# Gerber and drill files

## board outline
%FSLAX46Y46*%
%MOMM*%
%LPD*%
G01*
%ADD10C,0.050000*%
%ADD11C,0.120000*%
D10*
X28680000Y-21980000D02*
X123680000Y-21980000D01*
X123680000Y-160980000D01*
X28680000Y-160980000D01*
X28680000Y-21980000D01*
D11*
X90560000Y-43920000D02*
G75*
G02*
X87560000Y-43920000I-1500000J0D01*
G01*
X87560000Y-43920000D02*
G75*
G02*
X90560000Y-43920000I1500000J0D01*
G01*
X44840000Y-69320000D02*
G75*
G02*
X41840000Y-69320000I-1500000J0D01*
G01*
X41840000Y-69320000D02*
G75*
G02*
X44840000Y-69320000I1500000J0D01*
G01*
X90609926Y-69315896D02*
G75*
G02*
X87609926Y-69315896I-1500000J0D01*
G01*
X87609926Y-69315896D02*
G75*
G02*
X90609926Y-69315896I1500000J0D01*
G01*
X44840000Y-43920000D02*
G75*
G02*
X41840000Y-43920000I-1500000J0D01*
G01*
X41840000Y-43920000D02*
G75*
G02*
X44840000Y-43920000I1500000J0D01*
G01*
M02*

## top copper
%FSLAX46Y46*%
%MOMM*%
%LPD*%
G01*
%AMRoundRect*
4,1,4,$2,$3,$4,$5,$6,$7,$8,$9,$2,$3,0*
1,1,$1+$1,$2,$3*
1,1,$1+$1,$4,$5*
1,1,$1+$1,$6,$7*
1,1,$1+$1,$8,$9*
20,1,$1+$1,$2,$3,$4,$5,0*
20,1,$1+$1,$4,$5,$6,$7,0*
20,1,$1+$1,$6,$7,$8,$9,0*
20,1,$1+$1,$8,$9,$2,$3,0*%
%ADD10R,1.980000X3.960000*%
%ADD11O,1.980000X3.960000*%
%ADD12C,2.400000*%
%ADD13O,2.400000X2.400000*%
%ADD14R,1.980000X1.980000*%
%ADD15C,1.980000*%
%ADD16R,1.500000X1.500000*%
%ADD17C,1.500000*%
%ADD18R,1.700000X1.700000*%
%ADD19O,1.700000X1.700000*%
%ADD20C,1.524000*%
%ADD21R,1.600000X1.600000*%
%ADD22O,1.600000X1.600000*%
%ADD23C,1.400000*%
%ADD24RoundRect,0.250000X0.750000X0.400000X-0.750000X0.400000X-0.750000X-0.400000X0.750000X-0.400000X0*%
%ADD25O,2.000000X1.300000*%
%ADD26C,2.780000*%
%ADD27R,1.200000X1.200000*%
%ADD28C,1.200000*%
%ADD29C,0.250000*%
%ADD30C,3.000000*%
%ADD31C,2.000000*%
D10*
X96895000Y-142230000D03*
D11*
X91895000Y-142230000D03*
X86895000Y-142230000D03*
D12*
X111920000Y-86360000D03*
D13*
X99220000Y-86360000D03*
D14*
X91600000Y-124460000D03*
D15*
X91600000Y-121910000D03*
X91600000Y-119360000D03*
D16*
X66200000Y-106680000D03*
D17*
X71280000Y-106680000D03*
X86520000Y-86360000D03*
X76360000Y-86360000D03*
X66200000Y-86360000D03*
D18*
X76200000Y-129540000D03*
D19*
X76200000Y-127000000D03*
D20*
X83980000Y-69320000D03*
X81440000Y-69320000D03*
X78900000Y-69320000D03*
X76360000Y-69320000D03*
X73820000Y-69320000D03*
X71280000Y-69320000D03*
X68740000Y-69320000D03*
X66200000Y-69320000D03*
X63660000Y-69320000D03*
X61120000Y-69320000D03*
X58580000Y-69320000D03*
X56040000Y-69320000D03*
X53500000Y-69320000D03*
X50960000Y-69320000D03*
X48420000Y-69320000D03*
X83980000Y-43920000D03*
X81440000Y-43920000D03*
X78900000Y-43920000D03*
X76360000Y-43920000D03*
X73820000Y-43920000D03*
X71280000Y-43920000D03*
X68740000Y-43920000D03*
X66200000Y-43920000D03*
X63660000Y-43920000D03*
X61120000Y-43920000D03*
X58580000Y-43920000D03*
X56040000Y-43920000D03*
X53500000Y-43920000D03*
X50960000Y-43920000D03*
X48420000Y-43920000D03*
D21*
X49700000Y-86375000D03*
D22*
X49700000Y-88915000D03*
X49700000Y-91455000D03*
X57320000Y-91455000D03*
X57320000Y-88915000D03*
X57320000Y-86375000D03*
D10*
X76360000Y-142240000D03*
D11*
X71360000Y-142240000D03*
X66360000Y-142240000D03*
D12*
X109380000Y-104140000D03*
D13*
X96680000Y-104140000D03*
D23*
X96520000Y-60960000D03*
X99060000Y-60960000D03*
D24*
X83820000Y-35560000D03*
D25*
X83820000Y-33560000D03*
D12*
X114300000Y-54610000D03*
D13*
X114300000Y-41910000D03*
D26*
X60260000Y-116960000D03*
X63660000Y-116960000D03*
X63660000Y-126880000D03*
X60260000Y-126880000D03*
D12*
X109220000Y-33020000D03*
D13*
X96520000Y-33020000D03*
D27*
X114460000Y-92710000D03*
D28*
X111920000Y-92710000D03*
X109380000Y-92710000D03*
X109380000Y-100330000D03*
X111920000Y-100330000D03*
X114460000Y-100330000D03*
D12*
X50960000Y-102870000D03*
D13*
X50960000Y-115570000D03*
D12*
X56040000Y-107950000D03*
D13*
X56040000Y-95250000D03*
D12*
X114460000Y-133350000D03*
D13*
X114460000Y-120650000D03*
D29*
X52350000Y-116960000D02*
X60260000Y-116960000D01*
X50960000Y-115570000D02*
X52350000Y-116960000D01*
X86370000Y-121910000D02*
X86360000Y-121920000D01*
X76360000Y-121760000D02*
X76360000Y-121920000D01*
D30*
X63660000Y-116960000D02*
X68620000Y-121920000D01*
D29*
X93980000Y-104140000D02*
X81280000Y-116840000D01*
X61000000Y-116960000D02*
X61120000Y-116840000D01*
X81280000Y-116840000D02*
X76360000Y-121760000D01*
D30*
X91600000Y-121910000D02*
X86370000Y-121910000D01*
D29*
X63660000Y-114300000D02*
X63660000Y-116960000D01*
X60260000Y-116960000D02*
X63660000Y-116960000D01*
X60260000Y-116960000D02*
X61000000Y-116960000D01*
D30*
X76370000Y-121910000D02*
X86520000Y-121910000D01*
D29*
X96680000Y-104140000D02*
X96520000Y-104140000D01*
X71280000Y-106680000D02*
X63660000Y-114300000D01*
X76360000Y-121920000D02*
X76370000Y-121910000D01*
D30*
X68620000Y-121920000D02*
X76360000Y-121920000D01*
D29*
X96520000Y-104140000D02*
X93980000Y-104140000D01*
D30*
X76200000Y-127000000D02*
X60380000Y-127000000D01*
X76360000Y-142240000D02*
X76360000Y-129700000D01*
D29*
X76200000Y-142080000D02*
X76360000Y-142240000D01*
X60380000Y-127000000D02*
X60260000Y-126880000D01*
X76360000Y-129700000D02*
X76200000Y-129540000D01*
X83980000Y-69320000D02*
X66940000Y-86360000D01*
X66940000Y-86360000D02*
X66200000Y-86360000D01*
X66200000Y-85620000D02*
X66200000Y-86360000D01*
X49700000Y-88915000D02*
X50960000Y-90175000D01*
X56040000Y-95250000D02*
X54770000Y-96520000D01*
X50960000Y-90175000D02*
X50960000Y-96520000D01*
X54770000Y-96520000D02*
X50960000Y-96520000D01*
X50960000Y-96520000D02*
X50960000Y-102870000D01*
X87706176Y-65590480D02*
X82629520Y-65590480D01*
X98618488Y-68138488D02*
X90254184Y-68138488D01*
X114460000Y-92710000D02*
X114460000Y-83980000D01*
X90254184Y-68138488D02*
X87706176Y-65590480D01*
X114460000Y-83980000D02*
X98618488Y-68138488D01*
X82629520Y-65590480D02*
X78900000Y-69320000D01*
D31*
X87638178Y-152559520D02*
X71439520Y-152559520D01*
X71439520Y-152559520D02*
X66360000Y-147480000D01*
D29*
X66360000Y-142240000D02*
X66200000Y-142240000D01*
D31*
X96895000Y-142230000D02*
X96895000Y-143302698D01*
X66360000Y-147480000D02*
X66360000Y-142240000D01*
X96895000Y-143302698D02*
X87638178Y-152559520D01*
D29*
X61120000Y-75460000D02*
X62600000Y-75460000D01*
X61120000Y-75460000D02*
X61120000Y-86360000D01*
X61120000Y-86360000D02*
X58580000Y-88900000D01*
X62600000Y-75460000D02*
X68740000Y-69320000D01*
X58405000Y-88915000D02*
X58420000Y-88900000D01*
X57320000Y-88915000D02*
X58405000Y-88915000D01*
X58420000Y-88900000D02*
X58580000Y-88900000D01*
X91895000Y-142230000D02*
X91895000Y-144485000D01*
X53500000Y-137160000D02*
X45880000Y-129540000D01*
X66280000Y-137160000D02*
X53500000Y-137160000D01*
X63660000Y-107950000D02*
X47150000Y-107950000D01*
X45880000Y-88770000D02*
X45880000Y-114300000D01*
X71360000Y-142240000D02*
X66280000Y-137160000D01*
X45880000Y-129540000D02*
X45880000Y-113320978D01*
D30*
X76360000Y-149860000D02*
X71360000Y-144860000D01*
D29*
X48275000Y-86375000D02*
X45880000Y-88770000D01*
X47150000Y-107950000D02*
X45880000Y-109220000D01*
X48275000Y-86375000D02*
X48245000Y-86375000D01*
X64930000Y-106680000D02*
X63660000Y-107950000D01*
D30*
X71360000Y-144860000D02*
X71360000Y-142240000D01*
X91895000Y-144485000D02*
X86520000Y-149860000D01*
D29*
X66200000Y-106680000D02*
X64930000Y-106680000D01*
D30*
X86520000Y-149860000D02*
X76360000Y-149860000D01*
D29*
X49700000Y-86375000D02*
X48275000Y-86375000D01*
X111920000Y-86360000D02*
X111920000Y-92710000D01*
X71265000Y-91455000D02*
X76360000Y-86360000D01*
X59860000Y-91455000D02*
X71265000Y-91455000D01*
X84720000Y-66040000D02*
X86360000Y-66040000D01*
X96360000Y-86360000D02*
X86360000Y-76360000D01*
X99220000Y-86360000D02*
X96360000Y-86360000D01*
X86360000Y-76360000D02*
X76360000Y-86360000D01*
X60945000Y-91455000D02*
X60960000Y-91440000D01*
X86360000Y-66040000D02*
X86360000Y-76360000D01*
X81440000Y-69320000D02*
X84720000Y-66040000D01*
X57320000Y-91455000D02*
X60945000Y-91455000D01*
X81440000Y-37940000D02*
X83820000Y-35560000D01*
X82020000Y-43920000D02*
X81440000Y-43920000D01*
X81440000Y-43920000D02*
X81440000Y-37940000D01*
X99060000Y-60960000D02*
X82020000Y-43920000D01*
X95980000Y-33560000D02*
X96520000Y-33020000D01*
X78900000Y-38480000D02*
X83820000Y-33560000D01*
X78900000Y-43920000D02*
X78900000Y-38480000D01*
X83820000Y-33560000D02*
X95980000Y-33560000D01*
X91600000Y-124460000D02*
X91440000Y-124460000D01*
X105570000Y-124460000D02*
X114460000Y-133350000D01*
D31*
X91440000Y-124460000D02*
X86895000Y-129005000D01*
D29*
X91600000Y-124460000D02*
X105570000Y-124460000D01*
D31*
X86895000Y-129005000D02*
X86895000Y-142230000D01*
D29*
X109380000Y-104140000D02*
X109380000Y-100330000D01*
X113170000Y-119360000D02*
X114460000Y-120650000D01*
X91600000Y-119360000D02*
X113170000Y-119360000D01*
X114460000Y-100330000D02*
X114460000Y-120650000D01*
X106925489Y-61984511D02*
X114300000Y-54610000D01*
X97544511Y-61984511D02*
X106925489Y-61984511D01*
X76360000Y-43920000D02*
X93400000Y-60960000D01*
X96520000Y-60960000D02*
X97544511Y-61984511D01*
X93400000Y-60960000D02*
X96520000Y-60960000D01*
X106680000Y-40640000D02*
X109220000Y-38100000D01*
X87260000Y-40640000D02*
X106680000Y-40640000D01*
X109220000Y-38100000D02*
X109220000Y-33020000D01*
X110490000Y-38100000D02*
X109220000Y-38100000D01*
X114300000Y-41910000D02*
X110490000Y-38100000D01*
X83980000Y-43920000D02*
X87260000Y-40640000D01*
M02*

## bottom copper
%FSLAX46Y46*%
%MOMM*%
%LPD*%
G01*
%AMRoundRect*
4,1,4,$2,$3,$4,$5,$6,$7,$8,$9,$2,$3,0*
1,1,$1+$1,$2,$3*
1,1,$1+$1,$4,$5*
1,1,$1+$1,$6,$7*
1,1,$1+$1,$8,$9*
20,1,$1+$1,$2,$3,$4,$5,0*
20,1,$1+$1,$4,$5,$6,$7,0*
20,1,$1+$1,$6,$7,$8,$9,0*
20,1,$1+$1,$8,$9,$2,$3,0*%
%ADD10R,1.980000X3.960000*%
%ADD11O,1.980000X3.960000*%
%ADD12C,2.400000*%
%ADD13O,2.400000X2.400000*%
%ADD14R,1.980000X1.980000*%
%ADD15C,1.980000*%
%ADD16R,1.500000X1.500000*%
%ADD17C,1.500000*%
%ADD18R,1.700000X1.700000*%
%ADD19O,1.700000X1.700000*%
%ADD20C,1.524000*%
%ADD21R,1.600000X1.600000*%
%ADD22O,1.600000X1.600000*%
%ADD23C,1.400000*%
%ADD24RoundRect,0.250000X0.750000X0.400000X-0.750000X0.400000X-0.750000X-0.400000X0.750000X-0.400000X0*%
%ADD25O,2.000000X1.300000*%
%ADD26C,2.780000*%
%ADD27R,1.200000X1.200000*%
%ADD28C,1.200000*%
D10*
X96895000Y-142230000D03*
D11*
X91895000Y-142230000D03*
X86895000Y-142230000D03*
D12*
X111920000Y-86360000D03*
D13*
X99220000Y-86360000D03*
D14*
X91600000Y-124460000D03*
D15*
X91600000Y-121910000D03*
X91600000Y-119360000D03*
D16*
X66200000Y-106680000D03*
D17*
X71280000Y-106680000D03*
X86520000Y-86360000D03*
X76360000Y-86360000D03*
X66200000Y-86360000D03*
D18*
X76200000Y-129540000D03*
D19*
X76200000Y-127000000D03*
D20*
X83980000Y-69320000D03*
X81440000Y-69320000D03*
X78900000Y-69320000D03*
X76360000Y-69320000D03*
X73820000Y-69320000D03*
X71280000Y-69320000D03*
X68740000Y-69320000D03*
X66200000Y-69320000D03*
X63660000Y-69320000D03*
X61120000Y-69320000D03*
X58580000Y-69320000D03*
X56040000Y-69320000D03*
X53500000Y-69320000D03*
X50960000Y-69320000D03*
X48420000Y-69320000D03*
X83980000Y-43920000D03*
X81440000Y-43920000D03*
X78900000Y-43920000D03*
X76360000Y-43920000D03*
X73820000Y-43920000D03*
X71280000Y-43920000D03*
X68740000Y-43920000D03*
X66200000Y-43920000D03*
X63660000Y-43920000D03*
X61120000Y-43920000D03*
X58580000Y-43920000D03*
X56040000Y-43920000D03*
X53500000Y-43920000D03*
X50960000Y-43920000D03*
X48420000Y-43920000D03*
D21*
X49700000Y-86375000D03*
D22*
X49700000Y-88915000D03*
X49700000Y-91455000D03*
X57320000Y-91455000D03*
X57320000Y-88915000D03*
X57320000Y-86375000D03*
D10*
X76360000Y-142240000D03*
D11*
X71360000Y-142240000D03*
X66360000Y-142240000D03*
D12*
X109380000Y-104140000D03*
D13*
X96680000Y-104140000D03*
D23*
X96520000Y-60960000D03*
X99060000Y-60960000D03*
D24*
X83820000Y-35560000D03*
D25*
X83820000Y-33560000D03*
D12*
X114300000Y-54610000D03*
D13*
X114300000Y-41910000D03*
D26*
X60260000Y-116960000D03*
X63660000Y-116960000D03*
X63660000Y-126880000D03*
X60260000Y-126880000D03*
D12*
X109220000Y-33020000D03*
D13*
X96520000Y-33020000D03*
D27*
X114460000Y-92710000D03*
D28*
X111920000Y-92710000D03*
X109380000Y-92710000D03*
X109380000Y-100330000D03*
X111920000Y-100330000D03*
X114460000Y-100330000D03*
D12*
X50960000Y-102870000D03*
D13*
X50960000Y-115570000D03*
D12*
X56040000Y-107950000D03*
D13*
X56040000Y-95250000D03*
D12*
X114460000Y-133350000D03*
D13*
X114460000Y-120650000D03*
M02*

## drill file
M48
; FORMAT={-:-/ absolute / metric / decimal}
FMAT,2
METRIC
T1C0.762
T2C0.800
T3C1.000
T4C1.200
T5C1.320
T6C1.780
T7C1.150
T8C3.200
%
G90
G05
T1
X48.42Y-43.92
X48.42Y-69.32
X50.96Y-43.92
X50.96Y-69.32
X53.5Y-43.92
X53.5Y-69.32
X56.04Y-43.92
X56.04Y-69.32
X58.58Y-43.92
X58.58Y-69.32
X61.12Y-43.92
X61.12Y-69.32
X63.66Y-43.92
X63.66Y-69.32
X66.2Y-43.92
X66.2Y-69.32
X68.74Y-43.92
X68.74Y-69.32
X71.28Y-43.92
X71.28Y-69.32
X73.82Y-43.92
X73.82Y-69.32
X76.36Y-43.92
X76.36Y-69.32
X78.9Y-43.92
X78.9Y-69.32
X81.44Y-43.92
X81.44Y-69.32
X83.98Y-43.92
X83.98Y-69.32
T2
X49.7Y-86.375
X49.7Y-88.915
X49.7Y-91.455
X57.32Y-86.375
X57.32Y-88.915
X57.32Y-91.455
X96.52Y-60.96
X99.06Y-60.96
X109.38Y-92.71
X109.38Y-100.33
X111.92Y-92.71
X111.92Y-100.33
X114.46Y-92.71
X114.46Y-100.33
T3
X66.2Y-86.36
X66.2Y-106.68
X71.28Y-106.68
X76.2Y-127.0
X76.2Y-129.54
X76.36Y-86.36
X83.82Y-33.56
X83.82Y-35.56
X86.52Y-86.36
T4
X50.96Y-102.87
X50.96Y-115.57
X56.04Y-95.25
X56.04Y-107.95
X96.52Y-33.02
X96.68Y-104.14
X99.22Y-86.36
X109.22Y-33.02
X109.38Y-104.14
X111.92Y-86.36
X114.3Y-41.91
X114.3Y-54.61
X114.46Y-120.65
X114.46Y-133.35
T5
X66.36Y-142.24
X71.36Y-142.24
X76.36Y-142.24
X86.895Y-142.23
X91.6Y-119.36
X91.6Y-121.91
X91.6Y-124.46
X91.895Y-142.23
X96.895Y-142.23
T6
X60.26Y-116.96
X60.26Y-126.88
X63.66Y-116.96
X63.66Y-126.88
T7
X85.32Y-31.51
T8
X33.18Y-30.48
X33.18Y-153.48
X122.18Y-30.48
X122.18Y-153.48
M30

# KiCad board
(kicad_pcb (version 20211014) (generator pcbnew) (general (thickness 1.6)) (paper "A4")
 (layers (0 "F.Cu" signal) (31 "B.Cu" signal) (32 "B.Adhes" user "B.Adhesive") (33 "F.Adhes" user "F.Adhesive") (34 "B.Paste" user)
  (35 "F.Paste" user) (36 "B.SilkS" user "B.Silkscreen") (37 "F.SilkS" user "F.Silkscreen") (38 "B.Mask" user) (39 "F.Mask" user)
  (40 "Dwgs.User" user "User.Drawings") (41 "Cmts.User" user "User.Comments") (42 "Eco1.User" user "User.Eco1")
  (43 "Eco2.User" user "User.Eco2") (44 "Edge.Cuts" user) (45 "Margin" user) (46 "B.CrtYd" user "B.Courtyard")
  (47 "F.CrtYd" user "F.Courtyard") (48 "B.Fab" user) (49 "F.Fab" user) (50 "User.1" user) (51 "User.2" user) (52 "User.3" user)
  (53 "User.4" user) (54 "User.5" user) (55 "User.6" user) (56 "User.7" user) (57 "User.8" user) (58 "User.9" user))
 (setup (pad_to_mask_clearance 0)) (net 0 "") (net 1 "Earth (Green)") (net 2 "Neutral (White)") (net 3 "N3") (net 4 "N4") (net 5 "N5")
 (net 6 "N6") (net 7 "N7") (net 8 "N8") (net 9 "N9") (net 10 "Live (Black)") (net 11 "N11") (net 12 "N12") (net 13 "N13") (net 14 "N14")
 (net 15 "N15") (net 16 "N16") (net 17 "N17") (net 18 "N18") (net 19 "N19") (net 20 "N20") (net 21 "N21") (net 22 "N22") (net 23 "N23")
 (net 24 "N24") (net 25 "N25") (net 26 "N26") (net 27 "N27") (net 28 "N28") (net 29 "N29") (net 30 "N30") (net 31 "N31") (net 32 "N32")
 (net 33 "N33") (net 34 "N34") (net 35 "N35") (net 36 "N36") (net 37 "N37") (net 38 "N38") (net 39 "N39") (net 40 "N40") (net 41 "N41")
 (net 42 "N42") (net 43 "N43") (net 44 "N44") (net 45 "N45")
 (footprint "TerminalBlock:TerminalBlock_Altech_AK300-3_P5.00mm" (layer "F.Cu") (at 96.895 142.23 180)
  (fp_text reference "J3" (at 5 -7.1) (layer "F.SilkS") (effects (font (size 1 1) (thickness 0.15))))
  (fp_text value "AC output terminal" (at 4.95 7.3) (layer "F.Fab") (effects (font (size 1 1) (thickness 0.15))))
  (pad "1" thru_hole rect (at 0 0 180) (size 1.98 3.96) (drill 1.32) (layers *.Cu *.Mask) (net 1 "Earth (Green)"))
  (pad "2" thru_hole oval (at 5 0 180) (size 1.98 3.96) (drill 1.32) (layers *.Cu *.Mask) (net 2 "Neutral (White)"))
  (pad "3" thru_hole oval (at 10 0 180) (size 1.98 3.96) (drill 1.32) (layers *.Cu *.Mask) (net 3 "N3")))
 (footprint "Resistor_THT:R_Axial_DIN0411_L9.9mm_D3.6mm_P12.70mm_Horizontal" (layer "F.Cu") (at 111.92 86.36 180)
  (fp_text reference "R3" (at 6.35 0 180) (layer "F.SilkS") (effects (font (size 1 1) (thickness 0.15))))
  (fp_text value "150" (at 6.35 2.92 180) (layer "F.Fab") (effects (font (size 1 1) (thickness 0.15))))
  (pad "1" thru_hole circle (at 0 0 180) (size 2.4 2.4) (drill 1.2) (layers *.Cu *.Mask) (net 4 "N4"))
  (pad "2" thru_hole oval (at 12.7 0 180) (size 2.4 2.4) (drill 1.2) (layers *.Cu *.Mask) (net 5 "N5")))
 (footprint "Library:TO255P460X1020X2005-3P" (layer "F.Cu") (at 91.6 124.46 90)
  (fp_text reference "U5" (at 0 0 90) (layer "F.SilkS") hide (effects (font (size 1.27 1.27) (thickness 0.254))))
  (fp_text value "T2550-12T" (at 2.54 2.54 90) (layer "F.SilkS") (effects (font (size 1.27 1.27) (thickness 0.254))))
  (pad "1" thru_hole rect (at 0 0 90) (size 1.98 1.98) (drill 1.32) (layers *.Cu *.Mask) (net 3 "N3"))
  (pad "2" thru_hole circle (at 2.55 0 90) (size 1.98 1.98) (drill 1.32) (layers *.Cu *.Mask) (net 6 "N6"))
  (pad "3" thru_hole circle (at 5.1 0 90) (size 1.98 1.98) (drill 1.32) (layers *.Cu *.Mask) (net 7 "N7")))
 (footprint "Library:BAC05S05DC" (layer "F.Cu") (at 66.2 106.68 90)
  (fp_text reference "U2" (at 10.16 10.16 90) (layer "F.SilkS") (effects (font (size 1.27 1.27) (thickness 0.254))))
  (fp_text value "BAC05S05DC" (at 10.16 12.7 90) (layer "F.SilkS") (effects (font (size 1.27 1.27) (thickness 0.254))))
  (pad "1" thru_hole rect (at 0 0 90) (size 1.5 1.5) (drill 1) (layers *.Cu *.Mask) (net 2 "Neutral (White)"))
  (pad "2" thru_hole circle (at 0 5.08 90) (size 1.5 1.5) (drill 1) (layers *.Cu *.Mask) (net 6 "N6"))
  (pad "3" thru_hole circle (at 20.32 20.32 90) (size 1.5 1.5) (drill 1) (layers *.Cu *.Mask) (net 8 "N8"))
  (pad "4" thru_hole circle (at 20.32 10.16 90) (size 1.5 1.5) (drill 1) (layers *.Cu *.Mask) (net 5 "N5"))
  (pad "5" thru_hole circle (at 20.32 0 90) (size 1.5 1.5) (drill 1) (layers *.Cu *.Mask) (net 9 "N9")))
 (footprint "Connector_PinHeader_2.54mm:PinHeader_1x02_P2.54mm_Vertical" (layer "F.Cu") (at 76.2 129.54 180)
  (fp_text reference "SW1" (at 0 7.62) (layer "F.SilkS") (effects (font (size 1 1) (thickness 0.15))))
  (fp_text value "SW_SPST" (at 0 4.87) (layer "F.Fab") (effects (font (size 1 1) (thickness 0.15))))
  (pad "1" thru_hole rect (at 0 0 180) (size 1.7 1.7) (drill 1) (layers *.Cu *.Mask) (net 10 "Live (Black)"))
  (pad "2" thru_hole oval (at 0 2.54 180) (size 1.7 1.7) (drill 1) (layers *.Cu *.Mask) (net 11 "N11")))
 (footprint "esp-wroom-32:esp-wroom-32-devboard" (layer "F.Cu") (at 66.2 55.88 -90)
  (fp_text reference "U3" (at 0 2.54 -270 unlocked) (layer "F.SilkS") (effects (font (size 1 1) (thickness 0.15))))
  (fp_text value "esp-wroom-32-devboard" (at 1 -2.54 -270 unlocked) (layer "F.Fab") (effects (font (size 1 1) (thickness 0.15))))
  (fp_circle (center -11.96 -22.86) (end -10.46 -22.86) (layer "Edge.Cuts") (width 0.12) (fill none))
  (fp_circle (center 13.44 22.86) (end 14.94 22.86) (layer "Edge.Cuts") (width 0.12) (fill none))
  (fp_circle (center 13.435896 -22.909926) (end 14.935896 -22.909926) (layer "Edge.Cuts") (width 0.12) (fill none))
  (fp_circle (center -11.96 22.86) (end -10.46 22.86) (layer "Edge.Cuts") (width 0.12) (fill none))
  (pad "1" thru_hole circle (at 13.44 -17.78 270) (size 1.524 1.524) (drill 0.762) (layers *.Cu *.Mask) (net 9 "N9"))
  (pad "2" thru_hole circle (at 13.44 -15.24 270) (size 1.524 1.524) (drill 0.762) (layers *.Cu *.Mask) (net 5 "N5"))
  (pad "3" thru_hole circle (at 13.44 -12.7 270) (size 1.524 1.524) (drill 0.762) (layers *.Cu *.Mask) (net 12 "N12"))
  (pad "4" thru_hole circle (at 13.44 -10.16 270) (size 1.524 1.524) (drill 0.762) (layers *.Cu *.Mask) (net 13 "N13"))
  (pad "5" thru_hole circle (at 13.44 -7.62 270) (size 1.524 1.524) (drill 0.762) (layers *.Cu *.Mask) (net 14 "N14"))
  (pad "6" thru_hole circle (at 13.44 -5.08 270) (size 1.524 1.524) (drill 0.762) (layers *.Cu *.Mask) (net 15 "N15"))
  (pad "7" thru_hole circle (at 13.44 -2.54 270) (size 1.524 1.524) (drill 0.762) (layers *.Cu *.Mask) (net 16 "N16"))
  (pad "8" thru_hole circle (at 13.44 0 270) (size 1.524 1.524) (drill 0.762) (layers *.Cu *.Mask) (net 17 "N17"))
  (pad "9" thru_hole circle (at 13.44 2.54 270) (size 1.524 1.524) (drill 0.762) (layers *.Cu *.Mask) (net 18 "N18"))
  (pad "10" thru_hole circle (at 13.44 5.08 270) (size 1.524 1.524) (drill 0.762) (layers *.Cu *.Mask) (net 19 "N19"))
  (pad "11" thru_hole circle (at 13.44 7.62 270) (size 1.524 1.524) (drill 0.762) (layers *.Cu *.Mask) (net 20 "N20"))
  (pad "12" thru_hole circle (at 13.44 10.16 270) (size 1.524 1.524) (drill 0.762) (layers *.Cu *.Mask) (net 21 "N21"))
  (pad "13" thru_hole circle (at 13.44 12.7 270) (size 1.524 1.524) (drill 0.762) (layers *.Cu *.Mask) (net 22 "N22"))
  (pad "14" thru_hole circle (at 13.44 15.24 270) (size 1.524 1.524) (drill 0.762) (layers *.Cu *.Mask) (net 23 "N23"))
  (pad "15" thru_hole circle (at 13.44 17.78 270) (size 1.524 1.524) (drill 0.762) (layers *.Cu *.Mask) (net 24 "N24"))
  (pad "16" thru_hole circle (at -11.96 -17.78 270) (size 1.524 1.524) (drill 0.762) (layers *.Cu *.Mask) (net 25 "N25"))
  (pad "17" thru_hole circle (at -11.96 -15.24 270) (size 1.524 1.524) (drill 0.762) (layers *.Cu *.Mask) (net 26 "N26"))
  (pad "18" thru_hole circle (at -11.96 -12.7 270) (size 1.524 1.524) (drill 0.762) (layers *.Cu *.Mask) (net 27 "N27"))
  (pad "19" thru_hole circle (at -11.96 -10.16 270) (size 1.524 1.524) (drill 0.762) (layers *.Cu *.Mask) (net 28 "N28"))
  (pad "20" thru_hole circle (at -11.96 -7.62 270) (size 1.524 1.524) (drill 0.762) (layers *.Cu *.Mask) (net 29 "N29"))
  (pad "21" thru_hole circle (at -11.96 -5.08 270) (size 1.524 1.524) (drill 0.762) (layers *.Cu *.Mask) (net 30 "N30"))
  (pad "22" thru_hole circle (at -11.96 -2.54 270) (size 1.524 1.524) (drill 0.762) (layers *.Cu *.Mask) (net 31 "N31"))
  (pad "23" thru_hole circle (at -11.96 0 270) (size 1.524 1.524) (drill 0.762) (layers *.Cu *.Mask) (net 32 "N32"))
  (pad "24" thru_hole circle (at -11.96 2.54 270) (size 1.524 1.524) (drill 0.762) (layers *.Cu *.Mask) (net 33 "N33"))
  (pad "25" thru_hole circle (at -11.96 5.08 270) (size 1.524 1.524) (drill 0.762) (layers *.Cu *.Mask) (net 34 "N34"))
  (pad "26" thru_hole circle (at -11.96 7.62 270) (size 1.524 1.524) (drill 0.762) (layers *.Cu *.Mask) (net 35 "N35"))
  (pad "27" thru_hole circle (at -11.96 10.16 270) (size 1.524 1.524) (drill 0.762) (layers *.Cu *.Mask) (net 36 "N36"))
  (pad "28" thru_hole circle (at -11.96 12.7 270) (size 1.524 1.524) (drill 0.762) (layers *.Cu *.Mask) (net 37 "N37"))
  (pad "29" thru_hole circle (at -11.96 15.24 270) (size 1.524 1.524) (drill 0.762) (layers *.Cu *.Mask) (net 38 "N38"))
  (pad "30" thru_hole circle (at -11.96 17.78 270) (size 1.524 1.524) (drill 0.762) (layers *.Cu *.Mask) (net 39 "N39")))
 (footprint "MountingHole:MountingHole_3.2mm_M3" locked (layer "F.Cu") (at 33.18 30.48)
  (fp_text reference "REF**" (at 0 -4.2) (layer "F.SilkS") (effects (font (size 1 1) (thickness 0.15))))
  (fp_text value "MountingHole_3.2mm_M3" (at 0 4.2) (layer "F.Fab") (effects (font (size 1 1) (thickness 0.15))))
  (pad "" np_thru_hole circle locked (at 0 0) (size 3.2 3.2) (drill 3.2) (layers *.Cu *.Mask)))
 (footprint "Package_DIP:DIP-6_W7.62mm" (layer "F.Cu") (at 49.7 86.375)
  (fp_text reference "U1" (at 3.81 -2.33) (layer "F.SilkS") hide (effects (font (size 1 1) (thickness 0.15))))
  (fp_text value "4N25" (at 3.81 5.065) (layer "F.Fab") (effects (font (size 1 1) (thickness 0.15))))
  (pad "1" thru_hole rect (at 0 0) (size 1.6 1.6) (drill 0.8) (layers *.Cu *.Mask) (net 2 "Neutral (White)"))
  (pad "2" thru_hole oval (at 0 2.54) (size 1.6 1.6) (drill 0.8) (layers *.Cu *.Mask) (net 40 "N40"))
  (pad "3" thru_hole oval (at 0 5.08) (size 1.6 1.6) (drill 0.8) (layers *.Cu *.Mask) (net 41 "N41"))
  (pad "4" thru_hole oval (at 7.62 5.08) (size 1.6 1.6) (drill 0.8) (layers *.Cu *.Mask) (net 5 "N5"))
  (pad "5" thru_hole oval (at 7.62 2.54) (size 1.6 1.6) (drill 0.8) (layers *.Cu *.Mask) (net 16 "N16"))
  (pad "6" thru_hole oval (at 7.62 0) (size 1.6 1.6) (drill 0.8) (layers *.Cu *.Mask) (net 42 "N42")))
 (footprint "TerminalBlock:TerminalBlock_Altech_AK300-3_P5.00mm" (layer "F.Cu") (at 76.36 142.24 180)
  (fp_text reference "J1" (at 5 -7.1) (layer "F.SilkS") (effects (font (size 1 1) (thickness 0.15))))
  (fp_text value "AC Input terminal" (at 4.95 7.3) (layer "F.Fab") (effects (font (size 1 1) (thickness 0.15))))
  (pad "1" thru_hole rect (at 0 0 180) (size 1.98 3.96) (drill 1.32) (layers *.Cu *.Mask) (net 10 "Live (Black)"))
  (pad "2" thru_hole oval (at 5 0 180) (size 1.98 3.96) (drill 1.32) (layers *.Cu *.Mask) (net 2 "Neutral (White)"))
  (pad "3" thru_hole oval (at 10 0 180) (size 1.98 3.96) (drill 1.32) (layers *.Cu *.Mask) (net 1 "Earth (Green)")))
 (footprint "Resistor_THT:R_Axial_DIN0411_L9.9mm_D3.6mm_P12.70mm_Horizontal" (layer "F.Cu") (at 109.38 104.14 180)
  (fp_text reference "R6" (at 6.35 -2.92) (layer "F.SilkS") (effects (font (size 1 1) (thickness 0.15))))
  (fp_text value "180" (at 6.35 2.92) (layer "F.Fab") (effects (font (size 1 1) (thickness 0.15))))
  (pad "1" thru_hole circle (at 0 0 180) (size 2.4 2.4) (drill 1.2) (layers *.Cu *.Mask) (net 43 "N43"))
  (pad "2" thru_hole oval (at 12.7 0 180) (size 2.4 2.4) (drill 1.2) (layers *.Cu *.Mask) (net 6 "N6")))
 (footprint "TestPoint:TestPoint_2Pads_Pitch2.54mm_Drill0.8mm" (layer "F.Cu") (at 96.52 60.96)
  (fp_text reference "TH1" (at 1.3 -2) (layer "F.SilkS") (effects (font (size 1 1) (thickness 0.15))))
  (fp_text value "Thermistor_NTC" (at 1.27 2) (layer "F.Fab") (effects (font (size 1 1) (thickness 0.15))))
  (pad "1" thru_hole circle (at 0 0) (size 1.4 1.4) (drill 0.8) (layers *.Cu *.Mask) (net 28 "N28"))
  (pad "2" thru_hole circle (at 2.54 0) (size 1.4 1.4) (drill 0.8) (layers *.Cu *.Mask) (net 26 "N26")))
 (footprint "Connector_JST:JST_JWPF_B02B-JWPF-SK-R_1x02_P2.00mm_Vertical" (layer "F.Cu") (at 83.82 35.56 180)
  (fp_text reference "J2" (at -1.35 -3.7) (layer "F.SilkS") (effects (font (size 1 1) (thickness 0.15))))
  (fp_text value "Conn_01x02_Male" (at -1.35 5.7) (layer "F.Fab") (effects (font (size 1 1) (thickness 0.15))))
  (pad "" np_thru_hole circle (at -1.5 4.05 180) (size 1.15 1.15) (drill 1.15) (layers *.Cu *.Mask))
  (pad "1" thru_hole roundrect (at 0 0 180) (size 2 1.3) (drill 1) (layers *.Cu *.Mask) (roundrect_rratio 0.192308) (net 26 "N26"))
  (pad "2" thru_hole oval (at 0 2 180) (size 2 1.3) (drill 1) (layers *.Cu *.Mask) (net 27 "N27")))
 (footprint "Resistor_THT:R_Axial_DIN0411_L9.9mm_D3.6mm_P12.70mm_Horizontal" (layer "F.Cu") (at 114.3 54.61 90)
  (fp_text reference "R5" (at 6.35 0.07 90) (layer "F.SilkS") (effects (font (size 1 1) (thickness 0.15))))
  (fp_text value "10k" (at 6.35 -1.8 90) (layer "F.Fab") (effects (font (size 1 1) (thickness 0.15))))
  (pad "1" thru_hole circle (at 0 0 90) (size 2.4 2.4) (drill 1.2) (layers *.Cu *.Mask) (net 28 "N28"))
  (pad "2" thru_hole oval (at 12.7 0 90) (size 2.4 2.4) (drill 1.2) (layers *.Cu *.Mask) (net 25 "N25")))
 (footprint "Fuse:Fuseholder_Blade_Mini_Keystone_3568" (layer "F.Cu") (at 63.66 116.96 -90)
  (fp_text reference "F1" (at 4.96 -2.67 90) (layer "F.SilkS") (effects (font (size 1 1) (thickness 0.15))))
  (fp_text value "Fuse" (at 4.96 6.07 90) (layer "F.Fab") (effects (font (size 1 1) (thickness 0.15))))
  (pad "1" thru_hole circle (at 0 3.4 270) (size 2.78 2.78) (drill 1.78) (layers *.Cu *.Mask) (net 6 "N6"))
  (pad "1" thru_hole circle (at 0 0 270) (size 2.78 2.78) (drill 1.78) (layers *.Cu *.Mask) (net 6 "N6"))
  (pad "2" thru_hole circle (at 9.92 0 270) (size 2.78 2.78) (drill 1.78) (layers *.Cu *.Mask) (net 11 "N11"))
  (pad "2" thru_hole circle (at 9.92 3.4 270) (size 2.78 2.78) (drill 1.78) (layers *.Cu *.Mask) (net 11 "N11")))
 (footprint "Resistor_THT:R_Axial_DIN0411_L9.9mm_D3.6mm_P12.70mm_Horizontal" (layer "F.Cu") (at 109.22 33.02 180)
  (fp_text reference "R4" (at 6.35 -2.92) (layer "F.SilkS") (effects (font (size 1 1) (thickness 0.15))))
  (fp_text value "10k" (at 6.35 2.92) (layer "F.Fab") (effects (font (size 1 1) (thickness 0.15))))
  (pad "1" thru_hole circle (at 0 0 180) (size 2.4 2.4) (drill 1.2) (layers *.Cu *.Mask) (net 25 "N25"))
  (pad "2" thru_hole oval (at 12.7 0 180) (size 2.4 2.4) (drill 1.2) (layers *.Cu *.Mask) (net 27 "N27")))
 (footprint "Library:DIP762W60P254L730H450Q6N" (layer "F.Cu") (at 111.92 96.52 -90)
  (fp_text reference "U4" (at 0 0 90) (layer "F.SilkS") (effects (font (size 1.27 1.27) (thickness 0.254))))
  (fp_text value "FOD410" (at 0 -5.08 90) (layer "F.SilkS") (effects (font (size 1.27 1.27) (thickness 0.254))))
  (pad "1" thru_hole rect (at -3.81 -2.54 270) (size 1.2 1.2) (drill 0.8) (layers *.Cu *.Mask) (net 12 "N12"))
  (pad "2" thru_hole circle (at -3.81 0 270) (size 1.2 1.2) (drill 0.8) (layers *.Cu *.Mask) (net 4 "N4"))
  (pad "3" thru_hole circle (at -3.81 2.54 270) (size 1.2 1.2) (drill 0.8) (layers *.Cu *.Mask) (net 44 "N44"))
  (pad "4" thru_hole circle (at 3.81 2.54 270) (size 1.2 1.2) (drill 0.8) (layers *.Cu *.Mask) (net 43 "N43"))
  (pad "5" thru_hole circle (at 3.81 0 270) (size 1.2 1.2) (drill 0.8) (layers *.Cu *.Mask) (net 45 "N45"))
  (pad "6" thru_hole circle (at 3.81 -2.54 270) (size 1.2 1.2) (drill 0.8) (layers *.Cu *.Mask) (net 7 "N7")))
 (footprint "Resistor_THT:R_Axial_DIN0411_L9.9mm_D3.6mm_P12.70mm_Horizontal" (layer "F.Cu") (at 50.96 102.87 -90)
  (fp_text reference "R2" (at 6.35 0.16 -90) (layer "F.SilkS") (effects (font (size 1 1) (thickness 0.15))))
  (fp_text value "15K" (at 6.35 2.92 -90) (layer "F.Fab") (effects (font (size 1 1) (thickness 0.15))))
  (pad "1" thru_hole circle (at 0 0 270) (size 2.4 2.4) (drill 1.2) (layers *.Cu *.Mask) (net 40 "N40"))
  (pad "2" thru_hole oval (at 12.7 0 270) (size 2.4 2.4) (drill 1.2) (layers *.Cu *.Mask) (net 6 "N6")))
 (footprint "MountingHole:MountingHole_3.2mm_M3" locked (layer "F.Cu") (at 122.18 30.48)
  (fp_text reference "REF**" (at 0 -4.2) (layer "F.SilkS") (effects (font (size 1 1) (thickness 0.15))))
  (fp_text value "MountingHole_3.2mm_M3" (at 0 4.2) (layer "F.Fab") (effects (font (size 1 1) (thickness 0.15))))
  (pad "" np_thru_hole circle locked (at 0 0) (size 3.2 3.2) (drill 3.2) (layers *.Cu *.Mask)))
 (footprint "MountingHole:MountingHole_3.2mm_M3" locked (layer "F.Cu") (at 33.18 153.48)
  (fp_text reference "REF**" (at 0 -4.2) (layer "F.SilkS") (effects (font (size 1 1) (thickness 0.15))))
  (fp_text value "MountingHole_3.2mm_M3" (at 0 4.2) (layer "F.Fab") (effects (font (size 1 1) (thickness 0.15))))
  (pad "" np_thru_hole circle locked (at 0 0) (size 3.2 3.2) (drill 3.2) (layers *.Cu *.Mask)))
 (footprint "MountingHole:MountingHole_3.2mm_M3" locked (layer "F.Cu") (at 122.18 153.48)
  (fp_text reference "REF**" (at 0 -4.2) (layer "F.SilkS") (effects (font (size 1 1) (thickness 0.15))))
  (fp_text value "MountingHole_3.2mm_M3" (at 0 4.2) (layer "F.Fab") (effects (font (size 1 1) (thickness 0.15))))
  (pad "" np_thru_hole circle locked (at 0 0) (size 3.2 3.2) (drill 3.2) (layers *.Cu *.Mask)))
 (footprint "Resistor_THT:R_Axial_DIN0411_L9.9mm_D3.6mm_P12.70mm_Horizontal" (layer "F.Cu") (at 56.04 107.95 90)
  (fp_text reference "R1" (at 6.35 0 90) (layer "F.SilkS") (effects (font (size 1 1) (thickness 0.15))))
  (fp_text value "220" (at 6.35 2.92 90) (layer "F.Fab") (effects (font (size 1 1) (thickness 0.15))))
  (pad "1" thru_hole circle (at 0 0 90) (size 2.4 2.4) (drill 1.2) (layers *.Cu *.Mask) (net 2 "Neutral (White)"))
  (pad "2" thru_hole oval (at 12.7 0 90) (size 2.4 2.4) (drill 1.2) (layers *.Cu *.Mask) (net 40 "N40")))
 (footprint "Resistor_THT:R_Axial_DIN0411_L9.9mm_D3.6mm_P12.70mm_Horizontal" (layer "F.Cu") (at 114.46 133.35 90)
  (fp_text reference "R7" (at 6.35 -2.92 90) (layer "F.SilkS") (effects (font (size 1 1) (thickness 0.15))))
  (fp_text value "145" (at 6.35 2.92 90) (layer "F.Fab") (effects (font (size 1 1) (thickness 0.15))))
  (pad "1" thru_hole circle (at 0 0 90) (size 2.4 2.4) (drill 1.2) (layers *.Cu *.Mask) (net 3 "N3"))
  (pad "2" thru_hole oval (at 12.7 0 90) (size 2.4 2.4) (drill 1.2) (layers *.Cu *.Mask) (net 7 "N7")))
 (gr_rect locked (start 28.68 21.98) (end 123.68 160.98) (layer "Edge.Cuts") (width 0.05) (fill none))
 (segment (start 52.35 116.96) (end 60.26 116.96) (width 0.25) (layer "F.Cu") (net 6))
 (segment (start 50.96 115.57) (end 52.35 116.96) (width 0.25) (layer "F.Cu") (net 6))
 (segment (start 86.37 121.91) (end 86.36 121.92) (width 0.25) (layer "F.Cu") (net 6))
 (segment (start 76.36 121.76) (end 76.36 121.92) (width 0.25) (layer "F.Cu") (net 6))
 (segment (start 63.66 116.96) (end 68.62 121.92) (width 3) (layer "F.Cu") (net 6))
 (segment (start 93.98 104.14) (end 81.28 116.84) (width 0.25) (layer "F.Cu") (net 6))
 (segment (start 61 116.96) (end 61.12 116.84) (width 0.25) (layer "F.Cu") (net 6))
 (segment (start 81.28 116.84) (end 76.36 121.76) (width 0.25) (layer "F.Cu") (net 6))
 (segment (start 91.6 121.91) (end 86.37 121.91) (width 3) (layer "F.Cu") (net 6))
 (segment (start 63.66 114.3) (end 63.66 116.96) (width 0.25) (layer "F.Cu") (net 6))
 (segment (start 60.26 116.96) (end 63.66 116.96) (width 0.25) (layer "F.Cu") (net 6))
 (segment (start 60.26 116.96) (end 61 116.96) (width 0.25) (layer "F.Cu") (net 6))
 (segment (start 76.37 121.91) (end 86.52 121.91) (width 3) (layer "F.Cu") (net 6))
 (segment (start 96.68 104.14) (end 96.52 104.14) (width 0.25) (layer "F.Cu") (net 6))
 (segment (start 71.28 106.68) (end 63.66 114.3) (width 0.25) (layer "F.Cu") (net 6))
 (segment (start 76.36 121.92) (end 76.37 121.91) (width 0.25) (layer "F.Cu") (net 6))
 (segment (start 68.62 121.92) (end 76.36 121.92) (width 3) (layer "F.Cu") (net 6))
 (segment (start 96.52 104.14) (end 93.98 104.14) (width 0.25) (layer "F.Cu") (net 6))
 (segment (start 76.2 127) (end 60.38 127) (width 3) (layer "F.Cu") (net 11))
 (segment (start 76.36 142.24) (end 76.36 129.7) (width 3) (layer "F.Cu") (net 11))
 (segment (start 76.2 142.08) (end 76.36 142.24) (width 0.25) (layer "F.Cu") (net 11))
 (segment (start 60.38 127) (end 60.26 126.88) (width 0.25) (layer "F.Cu") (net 11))
 (segment (start 76.36 129.7) (end 76.2 129.54) (width 0.25) (layer "F.Cu") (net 11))
 (segment (start 83.98 69.32) (end 66.94 86.36) (width 0.25) (layer "F.Cu") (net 9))
 (segment (start 66.94 86.36) (end 66.2 86.36) (width 0.25) (layer "F.Cu") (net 9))
 (segment (start 66.2 85.62) (end 66.2 86.36) (width 0.25) (layer "F.Cu") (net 9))
 (segment (start 49.7 88.915) (end 50.96 90.175) (width 0.25) (layer "F.Cu") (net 40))
 (segment (start 56.04 95.25) (end 54.77 96.52) (width 0.25) (layer "F.Cu") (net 40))
 (segment (start 50.96 90.175) (end 50.96 96.52) (width 0.25) (layer "F.Cu") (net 40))
 (segment (start 54.77 96.52) (end 50.96 96.52) (width 0.25) (layer "F.Cu") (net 40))
 (segment (start 50.96 96.52) (end 50.96 102.87) (width 0.25) (layer "F.Cu") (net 40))
 (segment (start 87.706176 65.59048) (end 82.62952 65.59048) (width 0.25) (layer "F.Cu") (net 12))
 (segment (start 98.618488 68.138488) (end 90.254184 68.138488) (width 0.25) (layer "F.Cu") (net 12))
 (segment (start 114.46 92.71) (end 114.46 83.98) (width 0.25) (layer "F.Cu") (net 12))
 (segment (start 90.254184 68.138488) (end 87.706176 65.59048) (width 0.25) (layer "F.Cu") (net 12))
 (segment (start 114.46 83.98) (end 98.618488 68.138488) (width 0.25) (layer "F.Cu") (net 12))
 (segment (start 82.62952 65.59048) (end 78.9 69.32) (width 0.25) (layer "F.Cu") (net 12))
 (segment (start 87.638178 152.55952) (end 71.43952 152.55952) (width 2) (layer "F.Cu") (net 1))
 (segment (start 71.43952 152.55952) (end 66.36 147.48) (width 2) (layer "F.Cu") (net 1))
 (segment (start 66.36 142.24) (end 66.2 142.24) (width 0.25) (layer "F.Cu") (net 1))
 (segment (start 96.895 142.23) (end 96.895 143.302698) (width 2) (layer "F.Cu") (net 1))
 (segment (start 66.36 147.48) (end 66.36 142.24) (width 2) (layer "F.Cu") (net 1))
 (segment (start 96.895 143.302698) (end 87.638178 152.55952) (width 2) (layer "F.Cu") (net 1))
 (segment (start 61.12 75.46) (end 62.6 75.46) (width 0.25) (layer "F.Cu") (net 16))
 (segment (start 61.12 75.46) (end 61.12 86.36) (width 0.25) (layer "F.Cu") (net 16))
 (segment (start 61.12 86.36) (end 58.58 88.9) (width 0.25) (layer "F.Cu") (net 16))
 (segment (start 62.6 75.46) (end 68.74 69.32) (width 0.25) (layer "F.Cu") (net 16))
 (segment (start 58.405 88.915) (end 58.42 88.9) (width 0.25) (layer "F.Cu") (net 16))
 (segment (start 57.32 88.915) (end 58.405 88.915) (width 0.25) (layer "F.Cu") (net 16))
 (segment (start 58.42 88.9) (end 58.58 88.9) (width 0.25) (layer "F.Cu") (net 16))
 (segment (start 91.895 142.23) (end 91.895 144.485) (width 0.25) (layer "F.Cu") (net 2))
 (segment (start 53.5 137.16) (end 45.88 129.54) (width 0.25) (layer "F.Cu") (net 2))
 (segment (start 66.28 137.16) (end 53.5 137.16) (width 0.25) (layer "F.Cu") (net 2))
 (segment (start 63.66 107.95) (end 47.15 107.95) (width 0.25) (layer "F.Cu") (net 2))
 (segment (start 45.88 88.77) (end 45.88 114.3) (width 0.25) (layer "F.Cu") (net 2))
 (segment (start 71.36 142.24) (end 66.28 137.16) (width 0.25) (layer "F.Cu") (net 2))
 (segment (start 45.88 129.54) (end 45.88 113.320978) (width 0.25) (layer "F.Cu") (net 2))
 (segment (start 76.36 149.86) (end 71.36 144.86) (width 3) (layer "F.Cu") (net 2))
 (segment (start 48.275 86.375) (end 45.88 88.77) (width 0.25) (layer "F.Cu") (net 2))
 (segment (start 47.15 107.95) (end 45.88 109.22) (width 0.25) (layer "F.Cu") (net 2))
 (segment (start 48.275 86.375) (end 48.245 86.375) (width 0.25) (layer "F.Cu") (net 2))
 (segment (start 64.93 106.68) (end 63.66 107.95) (width 0.25) (layer "F.Cu") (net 2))
 (segment (start 71.36 144.86) (end 71.36 142.24) (width 3) (layer "F.Cu") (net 2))
 (segment (start 91.895 144.485) (end 86.52 149.86) (width 3) (layer "F.Cu") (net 2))
 (segment (start 66.2 106.68) (end 64.93 106.68) (width 0.25) (layer "F.Cu") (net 2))
 (segment (start 86.52 149.86) (end 76.36 149.86) (width 3) (layer "F.Cu") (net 2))
 (segment (start 49.7 86.375) (end 48.275 86.375) (width 0.25) (layer "F.Cu") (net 2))
 (segment (start 111.92 86.36) (end 111.92 92.71) (width 0.25) (layer "F.Cu") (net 4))
 (segment (start 71.265 91.455) (end 76.36 86.36) (width 0.25) (layer "F.Cu") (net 5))
 (segment (start 59.86 91.455) (end 71.265 91.455) (width 0.25) (layer "F.Cu") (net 5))
 (segment (start 84.72 66.04) (end 86.36 66.04) (width 0.25) (layer "F.Cu") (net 5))
 (segment (start 96.36 86.36) (end 86.36 76.36) (width 0.25) (layer "F.Cu") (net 5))
 (segment (start 99.22 86.36) (end 96.36 86.36) (width 0.25) (layer "F.Cu") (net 5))
 (segment (start 86.36 76.36) (end 76.36 86.36) (width 0.25) (layer "F.Cu") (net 5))
 (segment (start 60.945 91.455) (end 60.96 91.44) (width 0.25) (layer "F.Cu") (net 5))
 (segment (start 86.36 66.04) (end 86.36 76.36) (width 0.25) (layer "F.Cu") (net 5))
 (segment (start 81.44 69.32) (end 84.72 66.04) (width 0.25) (layer "F.Cu") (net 5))
 (segment (start 57.32 91.455) (end 60.945 91.455) (width 0.25) (layer "F.Cu") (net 5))
 (segment (start 81.44 37.94) (end 83.82 35.56) (width 0.25) (layer "F.Cu") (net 26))
 (segment (start 82.02 43.92) (end 81.44 43.92) (width 0.25) (layer "F.Cu") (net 26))
 (segment (start 81.44 43.92) (end 81.44 37.94) (width 0.25) (layer "F.Cu") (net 26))
 (segment (start 99.06 60.96) (end 82.02 43.92) (width 0.25) (layer "F.Cu") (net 26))
 (segment (start 95.98 33.56) (end 96.52 33.02) (width 0.25) (layer "F.Cu") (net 27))
 (segment (start 78.9 38.48) (end 83.82 33.56) (width 0.25) (layer "F.Cu") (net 27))
 (segment (start 78.9 43.92) (end 78.9 38.48) (width 0.25) (layer "F.Cu") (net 27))
 (segment (start 83.82 33.56) (end 95.98 33.56) (width 0.25) (layer "F.Cu") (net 27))
 (segment (start 91.6 124.46) (end 91.44 124.46) (width 0.25) (layer "F.Cu") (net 3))
 (segment (start 105.57 124.46) (end 114.46 133.35) (width 0.25) (layer "F.Cu") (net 3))
 (segment (start 91.44 124.46) (end 86.895 129.005) (width 2) (layer "F.Cu") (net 3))
 (segment (start 91.6 124.46) (end 105.57 124.46) (width 0.25) (layer "F.Cu") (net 3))
 (segment (start 86.895 129.005) (end 86.895 142.23) (width 2) (layer "F.Cu") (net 3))
 (segment (start 109.38 104.14) (end 109.38 100.33) (width 0.25) (layer "F.Cu") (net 43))
 (segment (start 113.17 119.36) (end 114.46 120.65) (width 0.25) (layer "F.Cu") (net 7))
 (segment (start 91.6 119.36) (end 113.17 119.36) (width 0.25) (layer "F.Cu") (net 7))
 (segment (start 114.46 100.33) (end 114.46 120.65) (width 0.25) (layer "F.Cu") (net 7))
 (segment (start 106.925489 61.984511) (end 114.3 54.61) (width 0.25) (layer "F.Cu") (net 28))
 (segment (start 97.544511 61.984511) (end 106.925489 61.984511) (width 0.25) (layer "F.Cu") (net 28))
 (segment (start 76.36 43.92) (end 93.4 60.96) (width 0.25) (layer "F.Cu") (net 28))
 (segment (start 96.52 60.96) (end 97.544511 61.984511) (width 0.25) (layer "F.Cu") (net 28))
 (segment (start 93.4 60.96) (end 96.52 60.96) (width 0.25) (layer "F.Cu") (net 28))
 (segment (start 106.68 40.64) (end 109.22 38.1) (width 0.25) (layer "F.Cu") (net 25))
 (segment (start 87.26 40.64) (end 106.68 40.64) (width 0.25) (layer "F.Cu") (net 25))
 (segment (start 109.22 38.1) (end 109.22 33.02) (width 0.25) (layer "F.Cu") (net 25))
 (segment (start 110.49 38.1) (end 109.22 38.1) (width 0.25) (layer "F.Cu") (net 25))
 (segment (start 114.3 41.91) (end 110.49 38.1) (width 0.25) (layer "F.Cu") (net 25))
 (segment (start 83.98 43.92) (end 87.26 40.64) (width 0.25) (layer "F.Cu") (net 25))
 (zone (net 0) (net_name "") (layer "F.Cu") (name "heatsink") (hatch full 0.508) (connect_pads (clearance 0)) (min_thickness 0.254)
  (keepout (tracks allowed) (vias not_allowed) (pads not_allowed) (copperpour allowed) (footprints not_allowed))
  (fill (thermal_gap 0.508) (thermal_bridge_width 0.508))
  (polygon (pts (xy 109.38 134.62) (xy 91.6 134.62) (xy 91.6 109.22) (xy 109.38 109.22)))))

